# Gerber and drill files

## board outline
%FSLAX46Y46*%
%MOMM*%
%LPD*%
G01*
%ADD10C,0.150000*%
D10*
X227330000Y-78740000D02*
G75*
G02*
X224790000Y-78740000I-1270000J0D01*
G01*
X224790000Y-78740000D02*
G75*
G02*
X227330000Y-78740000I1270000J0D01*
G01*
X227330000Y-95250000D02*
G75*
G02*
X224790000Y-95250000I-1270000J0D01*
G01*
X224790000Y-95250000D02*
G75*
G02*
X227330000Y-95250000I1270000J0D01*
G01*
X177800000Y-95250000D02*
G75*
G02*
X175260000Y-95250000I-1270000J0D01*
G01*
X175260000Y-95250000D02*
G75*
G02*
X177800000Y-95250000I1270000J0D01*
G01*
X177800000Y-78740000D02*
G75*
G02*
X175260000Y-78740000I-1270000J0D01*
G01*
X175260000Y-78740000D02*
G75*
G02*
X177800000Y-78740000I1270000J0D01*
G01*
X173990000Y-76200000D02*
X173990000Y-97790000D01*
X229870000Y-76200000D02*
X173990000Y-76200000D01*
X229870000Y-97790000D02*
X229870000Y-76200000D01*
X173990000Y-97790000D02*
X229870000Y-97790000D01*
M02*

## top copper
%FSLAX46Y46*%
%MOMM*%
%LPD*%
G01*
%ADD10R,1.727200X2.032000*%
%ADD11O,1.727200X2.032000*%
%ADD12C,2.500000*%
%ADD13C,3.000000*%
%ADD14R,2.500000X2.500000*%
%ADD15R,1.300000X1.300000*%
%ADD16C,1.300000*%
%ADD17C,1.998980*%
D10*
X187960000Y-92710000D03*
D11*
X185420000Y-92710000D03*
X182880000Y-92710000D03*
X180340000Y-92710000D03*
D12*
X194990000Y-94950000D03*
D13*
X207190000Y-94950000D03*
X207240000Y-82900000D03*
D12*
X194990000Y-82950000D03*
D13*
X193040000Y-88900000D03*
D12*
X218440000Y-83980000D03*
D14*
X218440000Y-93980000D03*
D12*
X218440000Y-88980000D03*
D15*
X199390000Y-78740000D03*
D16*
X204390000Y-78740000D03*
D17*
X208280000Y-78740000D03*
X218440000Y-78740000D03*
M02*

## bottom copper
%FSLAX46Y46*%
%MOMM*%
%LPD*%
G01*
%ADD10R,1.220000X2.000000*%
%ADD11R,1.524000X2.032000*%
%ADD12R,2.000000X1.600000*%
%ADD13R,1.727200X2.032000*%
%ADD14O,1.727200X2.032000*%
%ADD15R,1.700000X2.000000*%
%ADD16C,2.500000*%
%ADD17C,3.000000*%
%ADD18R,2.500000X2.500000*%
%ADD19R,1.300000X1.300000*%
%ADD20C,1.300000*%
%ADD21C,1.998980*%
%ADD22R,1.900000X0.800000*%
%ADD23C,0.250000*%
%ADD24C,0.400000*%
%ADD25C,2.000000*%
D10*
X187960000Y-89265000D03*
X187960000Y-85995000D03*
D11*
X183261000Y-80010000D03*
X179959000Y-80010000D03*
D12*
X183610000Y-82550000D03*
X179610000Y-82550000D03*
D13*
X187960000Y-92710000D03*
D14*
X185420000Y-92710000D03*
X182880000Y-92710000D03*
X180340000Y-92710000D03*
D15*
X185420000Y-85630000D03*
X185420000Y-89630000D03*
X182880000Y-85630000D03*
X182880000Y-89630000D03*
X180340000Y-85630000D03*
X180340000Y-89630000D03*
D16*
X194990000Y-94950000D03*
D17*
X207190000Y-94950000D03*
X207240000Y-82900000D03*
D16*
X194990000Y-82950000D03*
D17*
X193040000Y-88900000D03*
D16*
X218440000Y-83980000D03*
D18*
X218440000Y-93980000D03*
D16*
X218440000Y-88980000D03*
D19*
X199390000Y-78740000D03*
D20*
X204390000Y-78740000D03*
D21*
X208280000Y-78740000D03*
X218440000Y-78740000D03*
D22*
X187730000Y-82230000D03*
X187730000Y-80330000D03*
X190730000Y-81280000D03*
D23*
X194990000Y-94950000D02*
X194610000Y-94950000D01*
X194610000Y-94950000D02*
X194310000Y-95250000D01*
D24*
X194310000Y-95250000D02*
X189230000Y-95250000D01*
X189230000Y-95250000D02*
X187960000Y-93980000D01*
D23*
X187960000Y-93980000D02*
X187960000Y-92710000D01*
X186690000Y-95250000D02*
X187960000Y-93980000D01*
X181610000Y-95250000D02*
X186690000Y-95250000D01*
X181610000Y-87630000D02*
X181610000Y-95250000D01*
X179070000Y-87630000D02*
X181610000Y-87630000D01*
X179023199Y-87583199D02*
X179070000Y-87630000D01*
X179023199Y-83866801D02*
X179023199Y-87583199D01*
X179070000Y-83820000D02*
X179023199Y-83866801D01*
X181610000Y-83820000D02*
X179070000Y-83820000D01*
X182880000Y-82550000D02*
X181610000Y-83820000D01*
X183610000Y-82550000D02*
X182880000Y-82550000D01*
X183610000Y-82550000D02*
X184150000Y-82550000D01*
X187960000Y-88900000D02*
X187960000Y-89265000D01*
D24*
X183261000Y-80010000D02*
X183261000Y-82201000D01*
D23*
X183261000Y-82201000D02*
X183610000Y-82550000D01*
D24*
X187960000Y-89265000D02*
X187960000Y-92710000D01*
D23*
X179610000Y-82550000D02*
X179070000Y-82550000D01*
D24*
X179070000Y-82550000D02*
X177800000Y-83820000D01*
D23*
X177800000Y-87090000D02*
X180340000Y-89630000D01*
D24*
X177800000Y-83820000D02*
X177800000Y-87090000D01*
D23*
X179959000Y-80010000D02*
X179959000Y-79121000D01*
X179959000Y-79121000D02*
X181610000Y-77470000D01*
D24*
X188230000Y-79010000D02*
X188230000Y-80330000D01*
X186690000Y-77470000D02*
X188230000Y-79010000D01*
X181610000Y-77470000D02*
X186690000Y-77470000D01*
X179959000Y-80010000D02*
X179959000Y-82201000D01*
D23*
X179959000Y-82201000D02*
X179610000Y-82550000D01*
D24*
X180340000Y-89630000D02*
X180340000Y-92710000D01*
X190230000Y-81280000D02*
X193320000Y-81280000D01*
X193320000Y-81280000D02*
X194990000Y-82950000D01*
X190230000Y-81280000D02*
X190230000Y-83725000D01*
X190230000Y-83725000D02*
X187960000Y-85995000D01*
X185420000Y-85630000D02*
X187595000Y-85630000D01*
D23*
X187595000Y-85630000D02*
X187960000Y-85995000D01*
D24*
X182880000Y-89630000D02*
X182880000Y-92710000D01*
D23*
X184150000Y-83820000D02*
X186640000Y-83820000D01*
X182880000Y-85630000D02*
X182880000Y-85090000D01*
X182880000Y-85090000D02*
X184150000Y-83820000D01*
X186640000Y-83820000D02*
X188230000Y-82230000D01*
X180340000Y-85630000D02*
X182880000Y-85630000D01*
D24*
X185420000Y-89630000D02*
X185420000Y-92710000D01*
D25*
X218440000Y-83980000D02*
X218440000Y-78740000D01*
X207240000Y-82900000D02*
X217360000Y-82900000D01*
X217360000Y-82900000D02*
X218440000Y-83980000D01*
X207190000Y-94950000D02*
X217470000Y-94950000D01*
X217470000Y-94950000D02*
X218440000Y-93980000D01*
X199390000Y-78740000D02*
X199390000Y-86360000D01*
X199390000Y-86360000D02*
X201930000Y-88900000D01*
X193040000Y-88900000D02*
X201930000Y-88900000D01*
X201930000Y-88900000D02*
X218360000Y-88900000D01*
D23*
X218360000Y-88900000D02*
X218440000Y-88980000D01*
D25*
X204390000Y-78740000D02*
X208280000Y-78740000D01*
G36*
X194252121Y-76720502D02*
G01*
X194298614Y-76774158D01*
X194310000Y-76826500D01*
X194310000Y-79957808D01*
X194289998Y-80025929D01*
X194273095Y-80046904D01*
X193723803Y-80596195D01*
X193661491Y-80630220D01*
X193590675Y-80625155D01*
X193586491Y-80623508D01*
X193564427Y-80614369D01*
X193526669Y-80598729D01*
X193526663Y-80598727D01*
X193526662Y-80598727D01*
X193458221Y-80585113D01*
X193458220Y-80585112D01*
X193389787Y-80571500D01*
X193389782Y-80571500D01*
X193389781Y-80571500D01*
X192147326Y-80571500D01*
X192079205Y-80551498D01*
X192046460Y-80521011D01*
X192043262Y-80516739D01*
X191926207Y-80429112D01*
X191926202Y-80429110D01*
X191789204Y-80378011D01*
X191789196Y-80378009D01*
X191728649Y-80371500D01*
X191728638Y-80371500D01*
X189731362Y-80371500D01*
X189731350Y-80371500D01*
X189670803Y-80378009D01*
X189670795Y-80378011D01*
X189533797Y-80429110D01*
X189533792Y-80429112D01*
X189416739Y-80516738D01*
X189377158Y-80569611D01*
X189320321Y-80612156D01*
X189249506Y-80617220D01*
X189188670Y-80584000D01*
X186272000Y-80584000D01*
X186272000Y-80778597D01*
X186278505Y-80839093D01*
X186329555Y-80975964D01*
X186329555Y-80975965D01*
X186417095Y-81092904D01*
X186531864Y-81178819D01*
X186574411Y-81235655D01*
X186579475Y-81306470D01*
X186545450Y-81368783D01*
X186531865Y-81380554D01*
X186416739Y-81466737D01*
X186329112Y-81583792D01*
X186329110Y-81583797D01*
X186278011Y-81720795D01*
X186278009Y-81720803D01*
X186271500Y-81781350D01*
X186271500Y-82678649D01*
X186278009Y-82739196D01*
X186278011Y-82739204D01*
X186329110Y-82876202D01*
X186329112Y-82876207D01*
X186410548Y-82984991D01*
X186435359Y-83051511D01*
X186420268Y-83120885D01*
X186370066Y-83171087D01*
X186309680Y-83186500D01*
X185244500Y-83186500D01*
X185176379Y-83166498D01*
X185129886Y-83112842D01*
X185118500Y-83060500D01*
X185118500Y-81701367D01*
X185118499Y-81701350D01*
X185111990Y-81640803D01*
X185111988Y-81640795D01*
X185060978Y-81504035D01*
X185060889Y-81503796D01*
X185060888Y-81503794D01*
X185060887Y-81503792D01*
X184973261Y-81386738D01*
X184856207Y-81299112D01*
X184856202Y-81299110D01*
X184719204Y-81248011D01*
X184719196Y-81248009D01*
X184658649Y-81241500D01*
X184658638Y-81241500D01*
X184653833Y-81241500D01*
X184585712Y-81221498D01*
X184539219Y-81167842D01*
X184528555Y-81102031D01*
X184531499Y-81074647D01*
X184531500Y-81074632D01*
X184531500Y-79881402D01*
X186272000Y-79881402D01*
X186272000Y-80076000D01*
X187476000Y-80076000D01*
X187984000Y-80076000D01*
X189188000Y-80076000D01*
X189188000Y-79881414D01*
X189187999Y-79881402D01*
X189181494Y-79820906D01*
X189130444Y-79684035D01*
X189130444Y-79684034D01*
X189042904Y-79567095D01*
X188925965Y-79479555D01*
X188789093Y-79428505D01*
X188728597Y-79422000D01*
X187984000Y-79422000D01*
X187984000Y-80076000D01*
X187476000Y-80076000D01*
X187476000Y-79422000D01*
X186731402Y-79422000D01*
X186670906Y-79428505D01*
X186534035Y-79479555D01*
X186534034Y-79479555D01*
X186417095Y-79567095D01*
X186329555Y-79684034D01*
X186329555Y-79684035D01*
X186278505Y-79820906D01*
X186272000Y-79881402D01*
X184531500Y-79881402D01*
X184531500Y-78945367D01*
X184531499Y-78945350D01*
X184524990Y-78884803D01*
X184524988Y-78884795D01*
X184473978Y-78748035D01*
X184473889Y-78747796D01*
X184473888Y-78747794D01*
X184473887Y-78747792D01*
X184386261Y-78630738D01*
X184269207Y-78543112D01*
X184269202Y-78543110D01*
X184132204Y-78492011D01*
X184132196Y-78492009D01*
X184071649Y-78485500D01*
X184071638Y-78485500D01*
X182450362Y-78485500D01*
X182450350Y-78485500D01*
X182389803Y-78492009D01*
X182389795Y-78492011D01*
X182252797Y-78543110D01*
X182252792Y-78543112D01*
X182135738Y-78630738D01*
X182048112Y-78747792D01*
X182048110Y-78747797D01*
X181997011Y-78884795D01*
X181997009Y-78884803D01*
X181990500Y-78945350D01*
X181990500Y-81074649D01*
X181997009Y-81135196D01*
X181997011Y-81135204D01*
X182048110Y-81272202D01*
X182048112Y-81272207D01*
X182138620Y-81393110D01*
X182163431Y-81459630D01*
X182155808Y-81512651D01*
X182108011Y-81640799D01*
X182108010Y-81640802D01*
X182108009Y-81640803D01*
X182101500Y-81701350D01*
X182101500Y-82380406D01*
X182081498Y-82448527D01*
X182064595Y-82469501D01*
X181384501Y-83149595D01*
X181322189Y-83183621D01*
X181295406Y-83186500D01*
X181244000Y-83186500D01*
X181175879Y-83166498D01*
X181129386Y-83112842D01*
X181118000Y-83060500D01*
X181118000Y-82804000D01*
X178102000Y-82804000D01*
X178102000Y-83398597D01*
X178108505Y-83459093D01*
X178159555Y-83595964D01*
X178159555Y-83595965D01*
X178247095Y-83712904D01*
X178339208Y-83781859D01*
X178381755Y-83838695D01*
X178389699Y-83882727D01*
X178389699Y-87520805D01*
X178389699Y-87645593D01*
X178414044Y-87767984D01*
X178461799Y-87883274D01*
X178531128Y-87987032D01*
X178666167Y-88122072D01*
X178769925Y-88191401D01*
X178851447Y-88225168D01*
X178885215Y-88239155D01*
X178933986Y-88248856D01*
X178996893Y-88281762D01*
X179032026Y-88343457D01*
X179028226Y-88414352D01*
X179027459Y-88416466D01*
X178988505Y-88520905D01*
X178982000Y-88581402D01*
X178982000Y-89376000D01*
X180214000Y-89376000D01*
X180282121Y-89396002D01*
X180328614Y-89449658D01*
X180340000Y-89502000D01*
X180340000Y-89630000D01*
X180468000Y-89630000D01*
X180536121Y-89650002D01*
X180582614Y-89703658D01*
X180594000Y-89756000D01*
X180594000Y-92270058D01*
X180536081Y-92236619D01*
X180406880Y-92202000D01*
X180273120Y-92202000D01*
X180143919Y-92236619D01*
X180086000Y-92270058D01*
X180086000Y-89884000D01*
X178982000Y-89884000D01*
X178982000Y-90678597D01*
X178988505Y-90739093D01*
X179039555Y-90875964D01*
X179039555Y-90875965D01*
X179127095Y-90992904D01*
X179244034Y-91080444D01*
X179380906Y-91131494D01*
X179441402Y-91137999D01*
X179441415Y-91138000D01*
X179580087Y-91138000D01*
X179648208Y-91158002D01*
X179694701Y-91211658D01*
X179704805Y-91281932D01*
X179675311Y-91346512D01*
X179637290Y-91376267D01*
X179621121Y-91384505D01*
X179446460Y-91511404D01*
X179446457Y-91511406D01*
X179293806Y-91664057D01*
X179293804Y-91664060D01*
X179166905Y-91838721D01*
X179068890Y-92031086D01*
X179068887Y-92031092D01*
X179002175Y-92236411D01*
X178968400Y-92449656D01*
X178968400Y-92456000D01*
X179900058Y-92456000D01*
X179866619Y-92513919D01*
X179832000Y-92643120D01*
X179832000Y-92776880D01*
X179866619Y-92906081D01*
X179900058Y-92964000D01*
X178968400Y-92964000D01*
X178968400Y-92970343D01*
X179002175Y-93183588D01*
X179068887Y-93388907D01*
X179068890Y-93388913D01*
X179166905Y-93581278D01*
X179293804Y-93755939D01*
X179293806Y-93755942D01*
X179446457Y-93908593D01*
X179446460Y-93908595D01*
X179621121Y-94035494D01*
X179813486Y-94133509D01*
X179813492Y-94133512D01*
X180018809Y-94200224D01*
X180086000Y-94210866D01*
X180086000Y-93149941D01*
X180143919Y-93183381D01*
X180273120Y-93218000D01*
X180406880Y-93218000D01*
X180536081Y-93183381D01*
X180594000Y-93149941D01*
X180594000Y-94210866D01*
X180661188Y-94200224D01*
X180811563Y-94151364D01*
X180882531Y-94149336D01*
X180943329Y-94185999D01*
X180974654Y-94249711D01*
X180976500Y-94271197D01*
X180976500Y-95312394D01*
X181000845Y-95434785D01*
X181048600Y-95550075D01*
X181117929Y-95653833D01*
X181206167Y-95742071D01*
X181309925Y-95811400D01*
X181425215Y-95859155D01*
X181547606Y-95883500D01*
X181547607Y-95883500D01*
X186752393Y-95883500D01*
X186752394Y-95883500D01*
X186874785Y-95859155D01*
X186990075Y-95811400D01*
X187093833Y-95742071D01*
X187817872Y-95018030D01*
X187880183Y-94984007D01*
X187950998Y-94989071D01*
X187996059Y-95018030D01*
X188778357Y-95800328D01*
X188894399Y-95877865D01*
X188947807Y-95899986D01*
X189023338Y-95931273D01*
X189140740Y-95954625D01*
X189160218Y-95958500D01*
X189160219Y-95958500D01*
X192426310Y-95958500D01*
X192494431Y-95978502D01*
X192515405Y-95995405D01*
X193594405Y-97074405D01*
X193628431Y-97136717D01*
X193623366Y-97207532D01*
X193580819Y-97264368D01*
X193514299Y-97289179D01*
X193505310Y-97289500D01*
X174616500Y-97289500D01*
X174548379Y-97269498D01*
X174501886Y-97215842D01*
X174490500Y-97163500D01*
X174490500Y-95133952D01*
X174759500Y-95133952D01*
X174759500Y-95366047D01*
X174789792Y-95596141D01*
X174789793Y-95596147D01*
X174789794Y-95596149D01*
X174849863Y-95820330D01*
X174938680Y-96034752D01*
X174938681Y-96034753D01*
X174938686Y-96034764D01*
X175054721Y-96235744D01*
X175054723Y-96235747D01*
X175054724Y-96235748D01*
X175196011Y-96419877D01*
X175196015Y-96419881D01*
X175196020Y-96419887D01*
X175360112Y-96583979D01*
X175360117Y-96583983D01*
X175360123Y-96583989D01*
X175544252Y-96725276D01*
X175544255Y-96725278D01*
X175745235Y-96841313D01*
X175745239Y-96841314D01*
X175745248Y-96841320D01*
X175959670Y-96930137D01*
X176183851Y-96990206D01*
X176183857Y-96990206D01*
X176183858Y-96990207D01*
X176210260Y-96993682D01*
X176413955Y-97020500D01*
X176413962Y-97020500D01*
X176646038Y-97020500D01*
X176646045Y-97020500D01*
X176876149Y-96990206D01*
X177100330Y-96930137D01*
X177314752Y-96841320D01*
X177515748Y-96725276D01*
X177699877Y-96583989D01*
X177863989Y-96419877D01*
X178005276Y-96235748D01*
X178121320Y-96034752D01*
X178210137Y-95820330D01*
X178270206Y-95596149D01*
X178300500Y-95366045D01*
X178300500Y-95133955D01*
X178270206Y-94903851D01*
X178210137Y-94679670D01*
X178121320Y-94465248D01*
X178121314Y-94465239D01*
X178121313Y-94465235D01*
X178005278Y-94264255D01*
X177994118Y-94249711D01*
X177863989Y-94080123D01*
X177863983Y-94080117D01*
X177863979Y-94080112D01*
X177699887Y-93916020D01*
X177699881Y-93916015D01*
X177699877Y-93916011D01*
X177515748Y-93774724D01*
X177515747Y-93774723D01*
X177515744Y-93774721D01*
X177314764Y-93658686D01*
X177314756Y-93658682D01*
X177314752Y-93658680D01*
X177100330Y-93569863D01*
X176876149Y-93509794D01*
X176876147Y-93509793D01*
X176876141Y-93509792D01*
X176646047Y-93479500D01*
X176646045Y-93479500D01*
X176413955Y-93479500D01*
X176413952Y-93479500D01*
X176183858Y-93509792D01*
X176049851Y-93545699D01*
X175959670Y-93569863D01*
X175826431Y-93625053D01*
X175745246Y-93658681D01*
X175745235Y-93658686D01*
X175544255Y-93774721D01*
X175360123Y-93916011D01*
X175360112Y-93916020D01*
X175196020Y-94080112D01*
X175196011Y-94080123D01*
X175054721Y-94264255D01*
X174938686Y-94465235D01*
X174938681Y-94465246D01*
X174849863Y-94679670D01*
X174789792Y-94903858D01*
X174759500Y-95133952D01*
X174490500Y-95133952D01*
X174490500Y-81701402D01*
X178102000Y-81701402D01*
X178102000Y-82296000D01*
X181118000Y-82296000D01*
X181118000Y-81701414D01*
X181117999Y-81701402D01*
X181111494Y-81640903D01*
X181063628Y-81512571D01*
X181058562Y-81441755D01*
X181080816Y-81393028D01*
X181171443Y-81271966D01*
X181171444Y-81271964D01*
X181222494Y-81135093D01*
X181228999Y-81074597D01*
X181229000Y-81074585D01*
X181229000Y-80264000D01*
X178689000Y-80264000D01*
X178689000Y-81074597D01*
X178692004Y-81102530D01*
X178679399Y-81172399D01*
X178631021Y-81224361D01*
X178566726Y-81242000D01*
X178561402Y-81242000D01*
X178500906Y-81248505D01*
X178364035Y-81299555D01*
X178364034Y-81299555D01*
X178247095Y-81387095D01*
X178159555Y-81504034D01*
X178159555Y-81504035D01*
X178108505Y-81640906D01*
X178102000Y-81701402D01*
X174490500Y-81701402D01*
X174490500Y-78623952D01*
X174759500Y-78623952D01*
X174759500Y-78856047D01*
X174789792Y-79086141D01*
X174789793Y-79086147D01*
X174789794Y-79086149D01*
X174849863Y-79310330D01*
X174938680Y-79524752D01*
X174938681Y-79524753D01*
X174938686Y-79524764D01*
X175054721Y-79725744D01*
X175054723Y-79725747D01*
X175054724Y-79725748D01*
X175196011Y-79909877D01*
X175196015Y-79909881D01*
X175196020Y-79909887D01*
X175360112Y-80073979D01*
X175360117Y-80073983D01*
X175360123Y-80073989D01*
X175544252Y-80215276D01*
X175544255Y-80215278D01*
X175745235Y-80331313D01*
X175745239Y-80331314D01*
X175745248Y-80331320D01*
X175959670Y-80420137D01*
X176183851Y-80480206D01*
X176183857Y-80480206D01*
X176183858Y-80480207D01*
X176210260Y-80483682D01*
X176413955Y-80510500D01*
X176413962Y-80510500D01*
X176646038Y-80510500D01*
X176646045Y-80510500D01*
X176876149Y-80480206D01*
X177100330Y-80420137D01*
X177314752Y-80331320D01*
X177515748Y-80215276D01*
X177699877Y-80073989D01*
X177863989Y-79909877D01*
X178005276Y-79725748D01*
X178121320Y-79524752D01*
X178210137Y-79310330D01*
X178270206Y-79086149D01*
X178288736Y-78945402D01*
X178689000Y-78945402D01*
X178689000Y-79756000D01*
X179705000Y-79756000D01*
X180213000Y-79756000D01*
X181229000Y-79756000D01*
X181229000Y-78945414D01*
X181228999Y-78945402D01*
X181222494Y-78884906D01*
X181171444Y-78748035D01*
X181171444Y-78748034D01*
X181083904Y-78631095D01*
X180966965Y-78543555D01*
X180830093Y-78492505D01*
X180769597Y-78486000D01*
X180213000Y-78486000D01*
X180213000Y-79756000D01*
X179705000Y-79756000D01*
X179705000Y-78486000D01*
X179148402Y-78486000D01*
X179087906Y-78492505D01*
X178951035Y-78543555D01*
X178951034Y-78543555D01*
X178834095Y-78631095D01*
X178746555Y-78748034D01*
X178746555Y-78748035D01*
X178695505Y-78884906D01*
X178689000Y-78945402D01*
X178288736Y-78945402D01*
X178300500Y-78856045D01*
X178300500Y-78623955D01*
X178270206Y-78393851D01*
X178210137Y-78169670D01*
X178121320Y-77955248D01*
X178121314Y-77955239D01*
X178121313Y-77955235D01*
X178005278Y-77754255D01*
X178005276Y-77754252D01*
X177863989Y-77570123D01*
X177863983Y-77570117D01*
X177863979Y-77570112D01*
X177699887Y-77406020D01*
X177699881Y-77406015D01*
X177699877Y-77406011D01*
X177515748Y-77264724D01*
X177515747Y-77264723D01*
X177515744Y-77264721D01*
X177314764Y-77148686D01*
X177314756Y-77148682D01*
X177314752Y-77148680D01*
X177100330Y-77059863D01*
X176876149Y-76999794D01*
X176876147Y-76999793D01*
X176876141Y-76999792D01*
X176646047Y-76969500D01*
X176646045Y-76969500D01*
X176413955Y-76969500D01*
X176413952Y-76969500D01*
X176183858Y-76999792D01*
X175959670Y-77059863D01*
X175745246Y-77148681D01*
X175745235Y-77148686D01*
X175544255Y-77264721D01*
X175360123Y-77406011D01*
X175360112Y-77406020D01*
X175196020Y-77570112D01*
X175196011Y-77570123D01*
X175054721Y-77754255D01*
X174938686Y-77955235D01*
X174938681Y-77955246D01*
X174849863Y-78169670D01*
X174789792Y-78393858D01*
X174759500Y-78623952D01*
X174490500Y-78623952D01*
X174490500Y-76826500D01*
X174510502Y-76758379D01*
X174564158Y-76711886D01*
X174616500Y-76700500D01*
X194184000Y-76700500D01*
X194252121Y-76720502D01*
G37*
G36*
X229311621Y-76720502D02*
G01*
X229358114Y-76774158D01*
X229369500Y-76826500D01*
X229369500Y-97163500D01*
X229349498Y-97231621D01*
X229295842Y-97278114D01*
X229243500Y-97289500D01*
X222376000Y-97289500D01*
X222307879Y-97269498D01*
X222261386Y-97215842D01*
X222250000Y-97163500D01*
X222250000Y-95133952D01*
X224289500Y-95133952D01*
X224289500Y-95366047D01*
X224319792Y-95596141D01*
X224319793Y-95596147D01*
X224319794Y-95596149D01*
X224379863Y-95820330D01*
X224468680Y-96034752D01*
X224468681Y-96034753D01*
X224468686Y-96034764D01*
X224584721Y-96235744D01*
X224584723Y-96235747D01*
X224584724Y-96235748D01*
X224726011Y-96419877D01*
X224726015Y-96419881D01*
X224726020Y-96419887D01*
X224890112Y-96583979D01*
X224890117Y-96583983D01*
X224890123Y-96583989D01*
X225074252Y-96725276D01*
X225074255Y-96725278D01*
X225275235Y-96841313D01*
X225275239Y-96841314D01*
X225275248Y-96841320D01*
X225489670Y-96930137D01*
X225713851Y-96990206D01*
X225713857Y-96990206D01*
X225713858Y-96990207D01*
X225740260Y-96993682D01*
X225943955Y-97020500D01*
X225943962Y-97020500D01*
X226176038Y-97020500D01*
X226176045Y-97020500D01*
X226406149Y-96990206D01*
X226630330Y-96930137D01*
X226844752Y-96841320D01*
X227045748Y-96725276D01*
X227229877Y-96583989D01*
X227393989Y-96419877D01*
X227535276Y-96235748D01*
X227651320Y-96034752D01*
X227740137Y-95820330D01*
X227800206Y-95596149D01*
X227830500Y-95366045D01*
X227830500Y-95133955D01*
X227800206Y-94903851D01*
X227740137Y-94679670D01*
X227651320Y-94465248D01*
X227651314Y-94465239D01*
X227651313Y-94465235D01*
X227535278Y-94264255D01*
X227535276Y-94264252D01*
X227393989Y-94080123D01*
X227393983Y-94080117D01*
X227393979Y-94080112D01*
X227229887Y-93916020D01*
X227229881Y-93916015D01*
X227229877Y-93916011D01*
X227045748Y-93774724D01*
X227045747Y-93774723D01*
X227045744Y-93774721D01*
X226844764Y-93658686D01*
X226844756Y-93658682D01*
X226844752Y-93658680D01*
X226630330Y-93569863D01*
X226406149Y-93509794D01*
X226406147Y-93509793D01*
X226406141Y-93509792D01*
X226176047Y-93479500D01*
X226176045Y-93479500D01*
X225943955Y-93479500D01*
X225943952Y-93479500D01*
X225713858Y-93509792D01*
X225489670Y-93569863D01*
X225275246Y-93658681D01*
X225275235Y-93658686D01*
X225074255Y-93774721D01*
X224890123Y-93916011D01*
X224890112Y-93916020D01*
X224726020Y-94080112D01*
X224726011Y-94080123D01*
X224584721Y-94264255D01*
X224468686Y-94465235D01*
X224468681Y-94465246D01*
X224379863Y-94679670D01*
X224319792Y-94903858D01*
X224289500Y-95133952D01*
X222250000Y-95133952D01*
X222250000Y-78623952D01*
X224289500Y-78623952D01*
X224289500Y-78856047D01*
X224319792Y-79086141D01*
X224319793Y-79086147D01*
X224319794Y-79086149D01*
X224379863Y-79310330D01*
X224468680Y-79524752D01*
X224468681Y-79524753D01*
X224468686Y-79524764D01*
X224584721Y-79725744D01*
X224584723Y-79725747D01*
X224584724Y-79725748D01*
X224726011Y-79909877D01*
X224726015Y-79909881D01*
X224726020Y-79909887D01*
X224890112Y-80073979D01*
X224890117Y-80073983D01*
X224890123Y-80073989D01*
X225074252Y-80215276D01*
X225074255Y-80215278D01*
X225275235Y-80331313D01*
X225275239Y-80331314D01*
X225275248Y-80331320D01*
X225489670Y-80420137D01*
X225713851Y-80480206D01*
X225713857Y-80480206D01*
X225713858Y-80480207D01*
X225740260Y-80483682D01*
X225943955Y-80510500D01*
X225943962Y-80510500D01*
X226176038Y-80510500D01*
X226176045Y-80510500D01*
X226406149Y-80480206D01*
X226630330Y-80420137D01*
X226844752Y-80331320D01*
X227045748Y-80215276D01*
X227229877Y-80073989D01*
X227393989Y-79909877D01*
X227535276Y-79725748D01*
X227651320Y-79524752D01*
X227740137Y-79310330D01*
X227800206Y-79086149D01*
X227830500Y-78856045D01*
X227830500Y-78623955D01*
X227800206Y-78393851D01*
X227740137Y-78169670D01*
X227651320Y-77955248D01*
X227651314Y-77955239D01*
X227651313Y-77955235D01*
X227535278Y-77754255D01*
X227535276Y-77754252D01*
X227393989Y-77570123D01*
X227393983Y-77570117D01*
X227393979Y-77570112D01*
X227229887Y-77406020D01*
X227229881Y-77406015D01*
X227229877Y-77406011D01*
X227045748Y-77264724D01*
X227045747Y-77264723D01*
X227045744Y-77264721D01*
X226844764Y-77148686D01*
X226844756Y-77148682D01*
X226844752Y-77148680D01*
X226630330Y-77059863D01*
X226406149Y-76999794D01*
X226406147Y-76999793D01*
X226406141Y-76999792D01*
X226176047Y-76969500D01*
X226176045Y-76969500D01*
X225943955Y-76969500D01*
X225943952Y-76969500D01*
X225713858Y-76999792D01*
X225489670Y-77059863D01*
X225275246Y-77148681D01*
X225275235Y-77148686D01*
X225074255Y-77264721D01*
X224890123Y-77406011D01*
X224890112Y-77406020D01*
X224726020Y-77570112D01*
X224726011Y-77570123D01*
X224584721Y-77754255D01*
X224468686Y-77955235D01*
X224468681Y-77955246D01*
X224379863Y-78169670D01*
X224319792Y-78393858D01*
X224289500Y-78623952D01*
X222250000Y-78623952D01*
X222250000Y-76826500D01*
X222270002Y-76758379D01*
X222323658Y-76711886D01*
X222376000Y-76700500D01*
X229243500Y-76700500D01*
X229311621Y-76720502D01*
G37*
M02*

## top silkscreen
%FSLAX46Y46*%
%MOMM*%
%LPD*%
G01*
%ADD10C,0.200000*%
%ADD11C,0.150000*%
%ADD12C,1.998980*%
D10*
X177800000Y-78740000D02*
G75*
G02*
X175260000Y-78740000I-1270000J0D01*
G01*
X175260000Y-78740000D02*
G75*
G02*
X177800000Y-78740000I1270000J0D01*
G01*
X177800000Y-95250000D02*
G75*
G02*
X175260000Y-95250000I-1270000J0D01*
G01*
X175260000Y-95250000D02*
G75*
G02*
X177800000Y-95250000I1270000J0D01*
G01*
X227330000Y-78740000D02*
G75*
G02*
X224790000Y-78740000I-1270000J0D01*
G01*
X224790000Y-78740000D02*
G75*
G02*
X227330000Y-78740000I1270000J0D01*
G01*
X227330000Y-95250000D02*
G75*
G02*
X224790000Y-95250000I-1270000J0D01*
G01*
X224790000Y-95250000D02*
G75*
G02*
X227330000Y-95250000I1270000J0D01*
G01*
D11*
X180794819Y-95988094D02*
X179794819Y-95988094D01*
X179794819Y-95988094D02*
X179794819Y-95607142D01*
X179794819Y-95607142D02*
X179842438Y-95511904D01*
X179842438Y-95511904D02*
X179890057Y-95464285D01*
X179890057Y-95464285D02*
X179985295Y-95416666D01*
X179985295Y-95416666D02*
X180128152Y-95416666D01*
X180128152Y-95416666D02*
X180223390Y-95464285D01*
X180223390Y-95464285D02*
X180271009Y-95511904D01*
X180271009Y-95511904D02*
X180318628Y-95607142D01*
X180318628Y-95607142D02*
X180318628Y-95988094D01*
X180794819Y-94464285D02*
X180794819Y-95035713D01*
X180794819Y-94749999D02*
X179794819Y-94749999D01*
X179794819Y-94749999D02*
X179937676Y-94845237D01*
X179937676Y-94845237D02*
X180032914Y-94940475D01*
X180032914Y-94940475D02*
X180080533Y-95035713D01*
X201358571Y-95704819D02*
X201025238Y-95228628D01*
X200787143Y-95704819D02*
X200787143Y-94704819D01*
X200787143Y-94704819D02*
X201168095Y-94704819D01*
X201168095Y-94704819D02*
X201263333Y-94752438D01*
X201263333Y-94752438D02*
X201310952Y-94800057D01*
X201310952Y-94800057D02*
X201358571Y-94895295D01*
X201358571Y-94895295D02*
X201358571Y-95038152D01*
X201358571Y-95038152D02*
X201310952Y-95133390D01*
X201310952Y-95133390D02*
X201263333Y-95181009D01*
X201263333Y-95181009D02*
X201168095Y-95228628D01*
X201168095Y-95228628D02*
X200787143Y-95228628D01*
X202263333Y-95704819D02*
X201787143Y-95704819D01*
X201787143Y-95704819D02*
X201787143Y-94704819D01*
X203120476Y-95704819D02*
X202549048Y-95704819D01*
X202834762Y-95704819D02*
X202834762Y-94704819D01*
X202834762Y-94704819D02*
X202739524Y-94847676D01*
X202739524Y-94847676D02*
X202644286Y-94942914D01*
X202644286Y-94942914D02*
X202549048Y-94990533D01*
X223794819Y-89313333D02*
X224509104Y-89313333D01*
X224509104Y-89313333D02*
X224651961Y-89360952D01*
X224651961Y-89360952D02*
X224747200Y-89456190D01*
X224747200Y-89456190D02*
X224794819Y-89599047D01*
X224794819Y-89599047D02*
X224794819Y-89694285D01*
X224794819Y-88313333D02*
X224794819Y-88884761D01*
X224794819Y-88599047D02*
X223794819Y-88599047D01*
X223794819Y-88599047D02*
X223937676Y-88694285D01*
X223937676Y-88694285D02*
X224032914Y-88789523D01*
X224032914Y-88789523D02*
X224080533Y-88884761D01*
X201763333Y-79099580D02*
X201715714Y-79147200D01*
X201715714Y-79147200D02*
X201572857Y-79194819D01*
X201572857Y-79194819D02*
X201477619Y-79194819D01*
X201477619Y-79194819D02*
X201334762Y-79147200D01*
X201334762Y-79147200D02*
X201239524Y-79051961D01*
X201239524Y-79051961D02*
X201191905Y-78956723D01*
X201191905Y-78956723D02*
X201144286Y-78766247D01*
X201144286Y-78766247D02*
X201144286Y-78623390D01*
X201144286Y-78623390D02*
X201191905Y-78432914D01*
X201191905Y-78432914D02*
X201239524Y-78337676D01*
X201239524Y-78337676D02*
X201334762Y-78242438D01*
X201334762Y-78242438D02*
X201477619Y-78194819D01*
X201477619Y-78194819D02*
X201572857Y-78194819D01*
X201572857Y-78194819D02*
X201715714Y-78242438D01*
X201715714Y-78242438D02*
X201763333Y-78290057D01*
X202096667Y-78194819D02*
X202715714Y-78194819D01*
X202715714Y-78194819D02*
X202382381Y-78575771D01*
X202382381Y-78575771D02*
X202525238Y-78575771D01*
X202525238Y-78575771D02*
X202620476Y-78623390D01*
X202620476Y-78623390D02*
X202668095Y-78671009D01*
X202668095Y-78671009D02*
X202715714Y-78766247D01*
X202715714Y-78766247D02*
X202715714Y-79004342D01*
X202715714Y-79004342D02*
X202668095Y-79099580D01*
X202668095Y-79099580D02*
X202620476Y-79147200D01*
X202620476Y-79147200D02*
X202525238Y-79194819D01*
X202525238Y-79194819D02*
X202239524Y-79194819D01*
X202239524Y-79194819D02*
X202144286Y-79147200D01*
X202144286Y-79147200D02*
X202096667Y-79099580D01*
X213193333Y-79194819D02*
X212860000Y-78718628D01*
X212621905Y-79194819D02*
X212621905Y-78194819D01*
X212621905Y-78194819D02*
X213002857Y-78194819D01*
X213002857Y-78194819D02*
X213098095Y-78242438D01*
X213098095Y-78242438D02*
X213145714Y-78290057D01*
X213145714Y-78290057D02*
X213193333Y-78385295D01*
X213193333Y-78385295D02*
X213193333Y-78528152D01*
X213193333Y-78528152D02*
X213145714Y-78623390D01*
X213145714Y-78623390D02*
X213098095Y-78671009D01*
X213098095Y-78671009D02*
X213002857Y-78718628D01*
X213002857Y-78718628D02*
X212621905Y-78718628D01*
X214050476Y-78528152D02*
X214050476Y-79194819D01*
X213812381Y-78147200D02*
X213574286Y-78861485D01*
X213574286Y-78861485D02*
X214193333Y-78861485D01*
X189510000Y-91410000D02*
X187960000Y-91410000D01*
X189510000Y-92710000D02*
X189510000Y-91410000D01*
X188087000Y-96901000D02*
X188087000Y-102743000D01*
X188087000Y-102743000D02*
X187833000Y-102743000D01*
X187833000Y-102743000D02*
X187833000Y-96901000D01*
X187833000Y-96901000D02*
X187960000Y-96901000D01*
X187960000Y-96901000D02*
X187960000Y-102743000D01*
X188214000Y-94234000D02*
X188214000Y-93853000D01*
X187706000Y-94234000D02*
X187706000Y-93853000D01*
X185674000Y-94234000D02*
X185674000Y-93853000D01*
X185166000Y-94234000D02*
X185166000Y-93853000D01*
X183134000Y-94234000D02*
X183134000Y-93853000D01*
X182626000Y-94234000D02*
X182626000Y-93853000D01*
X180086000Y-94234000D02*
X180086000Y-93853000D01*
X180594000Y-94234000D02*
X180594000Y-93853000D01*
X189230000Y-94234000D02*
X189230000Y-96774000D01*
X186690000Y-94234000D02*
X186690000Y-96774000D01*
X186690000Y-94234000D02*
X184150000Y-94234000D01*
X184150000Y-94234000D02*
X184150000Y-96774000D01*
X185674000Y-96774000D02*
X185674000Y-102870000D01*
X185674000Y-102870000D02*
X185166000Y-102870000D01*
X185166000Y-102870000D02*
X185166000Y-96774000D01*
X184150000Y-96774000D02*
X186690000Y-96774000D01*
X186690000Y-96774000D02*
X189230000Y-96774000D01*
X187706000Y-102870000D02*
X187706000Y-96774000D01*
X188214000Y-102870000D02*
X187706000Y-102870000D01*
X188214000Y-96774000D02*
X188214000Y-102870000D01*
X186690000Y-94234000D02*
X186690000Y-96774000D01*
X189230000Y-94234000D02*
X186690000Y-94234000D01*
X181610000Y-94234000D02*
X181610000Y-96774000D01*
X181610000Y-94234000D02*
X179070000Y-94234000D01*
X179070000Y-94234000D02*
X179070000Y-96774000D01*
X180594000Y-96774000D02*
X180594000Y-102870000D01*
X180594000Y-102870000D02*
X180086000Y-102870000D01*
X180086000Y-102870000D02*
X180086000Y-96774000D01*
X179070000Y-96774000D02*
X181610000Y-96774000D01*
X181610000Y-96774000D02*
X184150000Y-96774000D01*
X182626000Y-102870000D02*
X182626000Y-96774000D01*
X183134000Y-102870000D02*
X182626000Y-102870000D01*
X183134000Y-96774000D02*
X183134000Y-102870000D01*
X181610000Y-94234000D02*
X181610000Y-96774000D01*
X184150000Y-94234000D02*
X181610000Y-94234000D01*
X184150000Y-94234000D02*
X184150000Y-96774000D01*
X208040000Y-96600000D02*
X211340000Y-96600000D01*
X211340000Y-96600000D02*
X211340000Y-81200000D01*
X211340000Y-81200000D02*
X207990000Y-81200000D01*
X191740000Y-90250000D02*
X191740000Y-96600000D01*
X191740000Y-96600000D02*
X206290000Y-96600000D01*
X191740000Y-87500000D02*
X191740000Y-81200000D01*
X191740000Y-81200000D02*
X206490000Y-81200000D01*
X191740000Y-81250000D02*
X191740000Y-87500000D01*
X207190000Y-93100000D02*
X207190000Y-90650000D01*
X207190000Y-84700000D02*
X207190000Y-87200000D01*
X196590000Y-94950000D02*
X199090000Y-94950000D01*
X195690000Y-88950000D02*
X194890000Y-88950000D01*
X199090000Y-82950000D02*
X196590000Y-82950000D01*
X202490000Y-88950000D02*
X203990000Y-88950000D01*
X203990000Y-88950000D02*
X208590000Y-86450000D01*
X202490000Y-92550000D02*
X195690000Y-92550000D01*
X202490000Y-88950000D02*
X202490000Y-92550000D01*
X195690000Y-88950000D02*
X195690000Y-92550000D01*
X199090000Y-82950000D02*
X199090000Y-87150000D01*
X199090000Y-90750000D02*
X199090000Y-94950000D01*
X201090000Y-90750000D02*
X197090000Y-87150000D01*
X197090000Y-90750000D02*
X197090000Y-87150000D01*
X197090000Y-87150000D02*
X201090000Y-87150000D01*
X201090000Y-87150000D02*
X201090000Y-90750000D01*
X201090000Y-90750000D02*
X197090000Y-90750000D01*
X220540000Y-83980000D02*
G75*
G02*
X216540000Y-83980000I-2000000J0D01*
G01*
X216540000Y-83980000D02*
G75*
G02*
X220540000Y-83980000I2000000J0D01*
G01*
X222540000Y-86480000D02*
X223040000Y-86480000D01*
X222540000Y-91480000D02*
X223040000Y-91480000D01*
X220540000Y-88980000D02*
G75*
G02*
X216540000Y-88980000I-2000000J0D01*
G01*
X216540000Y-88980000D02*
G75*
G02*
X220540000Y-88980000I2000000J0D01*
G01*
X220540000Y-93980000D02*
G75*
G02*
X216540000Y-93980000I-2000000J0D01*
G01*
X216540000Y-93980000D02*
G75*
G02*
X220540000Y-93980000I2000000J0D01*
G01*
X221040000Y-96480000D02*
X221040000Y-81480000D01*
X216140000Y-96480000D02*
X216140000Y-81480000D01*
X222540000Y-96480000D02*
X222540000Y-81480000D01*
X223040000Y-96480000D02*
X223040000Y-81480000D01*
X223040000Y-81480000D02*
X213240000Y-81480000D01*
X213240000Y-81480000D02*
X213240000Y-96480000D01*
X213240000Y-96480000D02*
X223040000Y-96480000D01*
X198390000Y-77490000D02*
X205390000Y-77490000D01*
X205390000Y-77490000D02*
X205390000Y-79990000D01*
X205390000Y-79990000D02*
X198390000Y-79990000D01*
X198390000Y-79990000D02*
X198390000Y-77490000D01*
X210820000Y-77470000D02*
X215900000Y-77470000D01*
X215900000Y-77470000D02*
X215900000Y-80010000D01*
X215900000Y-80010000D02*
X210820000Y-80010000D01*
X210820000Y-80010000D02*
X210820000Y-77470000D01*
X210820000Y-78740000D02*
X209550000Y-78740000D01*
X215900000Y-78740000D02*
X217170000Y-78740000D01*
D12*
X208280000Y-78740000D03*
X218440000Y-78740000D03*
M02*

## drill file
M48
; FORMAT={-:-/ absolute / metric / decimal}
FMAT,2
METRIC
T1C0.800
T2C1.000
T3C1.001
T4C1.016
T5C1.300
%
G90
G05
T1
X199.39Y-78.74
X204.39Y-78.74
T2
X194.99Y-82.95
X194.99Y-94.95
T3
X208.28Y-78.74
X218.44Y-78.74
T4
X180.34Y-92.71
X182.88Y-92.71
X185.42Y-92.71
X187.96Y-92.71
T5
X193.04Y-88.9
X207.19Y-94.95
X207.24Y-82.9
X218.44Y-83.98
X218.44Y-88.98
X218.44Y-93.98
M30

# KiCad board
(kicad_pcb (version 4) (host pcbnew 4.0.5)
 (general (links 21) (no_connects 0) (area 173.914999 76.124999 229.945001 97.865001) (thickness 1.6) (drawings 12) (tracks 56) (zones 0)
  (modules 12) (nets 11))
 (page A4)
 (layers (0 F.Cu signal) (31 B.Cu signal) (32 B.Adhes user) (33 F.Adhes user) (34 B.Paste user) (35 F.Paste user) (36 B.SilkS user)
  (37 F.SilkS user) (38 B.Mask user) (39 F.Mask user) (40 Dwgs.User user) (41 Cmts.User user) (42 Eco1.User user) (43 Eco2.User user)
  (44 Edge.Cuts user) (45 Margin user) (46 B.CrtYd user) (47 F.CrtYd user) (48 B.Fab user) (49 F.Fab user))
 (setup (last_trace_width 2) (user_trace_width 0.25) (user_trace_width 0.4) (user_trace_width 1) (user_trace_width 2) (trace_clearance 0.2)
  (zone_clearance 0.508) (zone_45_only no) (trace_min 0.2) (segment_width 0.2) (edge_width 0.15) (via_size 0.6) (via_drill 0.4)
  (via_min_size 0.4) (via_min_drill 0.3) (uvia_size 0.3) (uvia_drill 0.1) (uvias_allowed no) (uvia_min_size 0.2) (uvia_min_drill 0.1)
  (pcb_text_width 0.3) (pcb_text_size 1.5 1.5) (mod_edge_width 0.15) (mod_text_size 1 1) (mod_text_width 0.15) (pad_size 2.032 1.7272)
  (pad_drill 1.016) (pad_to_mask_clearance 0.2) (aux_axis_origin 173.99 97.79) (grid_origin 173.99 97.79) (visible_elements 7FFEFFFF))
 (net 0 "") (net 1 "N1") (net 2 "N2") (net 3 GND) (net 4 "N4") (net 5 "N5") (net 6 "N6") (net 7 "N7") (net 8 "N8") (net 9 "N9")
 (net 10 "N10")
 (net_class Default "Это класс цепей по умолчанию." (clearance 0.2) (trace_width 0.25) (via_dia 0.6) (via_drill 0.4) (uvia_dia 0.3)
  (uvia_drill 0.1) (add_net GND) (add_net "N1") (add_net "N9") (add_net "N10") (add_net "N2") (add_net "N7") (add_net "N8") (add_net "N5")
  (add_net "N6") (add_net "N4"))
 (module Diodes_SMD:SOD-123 (layer B.Cu) (at 187.96 87.63 90)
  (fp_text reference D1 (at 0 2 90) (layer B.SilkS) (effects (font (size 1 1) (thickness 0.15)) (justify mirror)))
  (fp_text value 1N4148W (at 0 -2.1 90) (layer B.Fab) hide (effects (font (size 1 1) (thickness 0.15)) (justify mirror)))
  (pad 1 smd rect (at -1.635 0 90) (size 2 1.22) (layers B.Cu B.Paste B.Mask) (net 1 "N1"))
  (pad 2 smd rect (at 1.635 0 90) (size 2 1.22) (layers B.Cu B.Paste B.Mask) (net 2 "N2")))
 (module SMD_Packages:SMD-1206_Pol (layer B.Cu) (at 181.61 80.01 180)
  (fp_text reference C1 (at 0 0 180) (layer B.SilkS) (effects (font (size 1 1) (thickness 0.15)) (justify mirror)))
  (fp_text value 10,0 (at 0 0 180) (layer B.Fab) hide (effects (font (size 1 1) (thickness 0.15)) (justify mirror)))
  (pad 1 smd rect (at -1.651 0 180) (size 1.524 2.032) (layers B.Cu B.Paste B.Mask) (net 1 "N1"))
  (pad 2 smd rect (at 1.651 0 180) (size 1.524 2.032) (layers B.Cu B.Paste B.Mask) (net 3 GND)))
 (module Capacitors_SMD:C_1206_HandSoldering (layer B.Cu) (at 181.61 82.55 180)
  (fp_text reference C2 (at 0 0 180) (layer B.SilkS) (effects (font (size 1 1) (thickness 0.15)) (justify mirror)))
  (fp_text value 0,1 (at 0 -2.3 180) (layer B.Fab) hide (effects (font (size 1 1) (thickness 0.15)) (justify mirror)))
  (pad 1 smd rect (at -2 0 180) (size 2 1.6) (layers B.Cu B.Paste B.Mask) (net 1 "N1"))
  (pad 2 smd rect (at 2 0 180) (size 2 1.6) (layers B.Cu B.Paste B.Mask) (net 3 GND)))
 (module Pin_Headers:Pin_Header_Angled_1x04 (layer F.Cu) (at 187.96 92.71 270)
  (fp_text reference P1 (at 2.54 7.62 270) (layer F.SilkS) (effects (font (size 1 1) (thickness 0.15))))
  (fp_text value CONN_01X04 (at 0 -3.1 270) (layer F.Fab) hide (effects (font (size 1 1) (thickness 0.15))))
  (fp_line (start -1.3 -1.55) (end -1.3 0) (layer F.SilkS) (width 0.15))
  (fp_line (start 0 -1.55) (end -1.3 -1.55) (layer F.SilkS) (width 0.15))
  (fp_line (start 4.191 -0.127) (end 10.033 -0.127) (layer F.SilkS) (width 0.15))
  (fp_line (start 10.033 -0.127) (end 10.033 0.127) (layer F.SilkS) (width 0.15))
  (fp_line (start 10.033 0.127) (end 4.191 0.127) (layer F.SilkS) (width 0.15))
  (fp_line (start 4.191 0.127) (end 4.191 0) (layer F.SilkS) (width 0.15))
  (fp_line (start 4.191 0) (end 10.033 0) (layer F.SilkS) (width 0.15))
  (fp_line (start 1.524 -0.254) (end 1.143 -0.254) (layer F.SilkS) (width 0.15))
  (fp_line (start 1.524 0.254) (end 1.143 0.254) (layer F.SilkS) (width 0.15))
  (fp_line (start 1.524 2.286) (end 1.143 2.286) (layer F.SilkS) (width 0.15))
  (fp_line (start 1.524 2.794) (end 1.143 2.794) (layer F.SilkS) (width 0.15))
  (fp_line (start 1.524 4.826) (end 1.143 4.826) (layer F.SilkS) (width 0.15))
  (fp_line (start 1.524 5.334) (end 1.143 5.334) (layer F.SilkS) (width 0.15))
  (fp_line (start 1.524 7.874) (end 1.143 7.874) (layer F.SilkS) (width 0.15))
  (fp_line (start 1.524 7.366) (end 1.143 7.366) (layer F.SilkS) (width 0.15))
  (fp_line (start 1.524 -1.27) (end 4.064 -1.27) (layer F.SilkS) (width 0.15))
  (fp_line (start 1.524 1.27) (end 4.064 1.27) (layer F.SilkS) (width 0.15))
  (fp_line (start 1.524 1.27) (end 1.524 3.81) (layer F.SilkS) (width 0.15))
  (fp_line (start 1.524 3.81) (end 4.064 3.81) (layer F.SilkS) (width 0.15))
  (fp_line (start 4.064 2.286) (end 10.16 2.286) (layer F.SilkS) (width 0.15))
  (fp_line (start 10.16 2.286) (end 10.16 2.794) (layer F.SilkS) (width 0.15))
  (fp_line (start 10.16 2.794) (end 4.064 2.794) (layer F.SilkS) (width 0.15))
  (fp_line (start 4.064 3.81) (end 4.064 1.27) (layer F.SilkS) (width 0.15))
  (fp_line (start 4.064 1.27) (end 4.064 -1.27) (layer F.SilkS) (width 0.15))
  (fp_line (start 10.16 0.254) (end 4.064 0.254) (layer F.SilkS) (width 0.15))
  (fp_line (start 10.16 -0.254) (end 10.16 0.254) (layer F.SilkS) (width 0.15))
  (fp_line (start 4.064 -0.254) (end 10.16 -0.254) (layer F.SilkS) (width 0.15))
  (fp_line (start 1.524 1.27) (end 4.064 1.27) (layer F.SilkS) (width 0.15))
  (fp_line (start 1.524 -1.27) (end 1.524 1.27) (layer F.SilkS) (width 0.15))
  (fp_line (start 1.524 6.35) (end 4.064 6.35) (layer F.SilkS) (width 0.15))
  (fp_line (start 1.524 6.35) (end 1.524 8.89) (layer F.SilkS) (width 0.15))
  (fp_line (start 1.524 8.89) (end 4.064 8.89) (layer F.SilkS) (width 0.15))
  (fp_line (start 4.064 7.366) (end 10.16 7.366) (layer F.SilkS) (width 0.15))
  (fp_line (start 10.16 7.366) (end 10.16 7.874) (layer F.SilkS) (width 0.15))
  (fp_line (start 10.16 7.874) (end 4.064 7.874) (layer F.SilkS) (width 0.15))
  (fp_line (start 4.064 8.89) (end 4.064 6.35) (layer F.SilkS) (width 0.15))
  (fp_line (start 4.064 6.35) (end 4.064 3.81) (layer F.SilkS) (width 0.15))
  (fp_line (start 10.16 5.334) (end 4.064 5.334) (layer F.SilkS) (width 0.15))
  (fp_line (start 10.16 4.826) (end 10.16 5.334) (layer F.SilkS) (width 0.15))
  (fp_line (start 4.064 4.826) (end 10.16 4.826) (layer F.SilkS) (width 0.15))
  (fp_line (start 1.524 6.35) (end 4.064 6.35) (layer F.SilkS) (width 0.15))
  (fp_line (start 1.524 3.81) (end 1.524 6.35) (layer F.SilkS) (width 0.15))
  (fp_line (start 1.524 3.81) (end 4.064 3.81) (layer F.SilkS) (width 0.15))
  (pad 1 thru_hole rect (at 0 0 270) (size 2.032 1.7272) (drill 1.016) (layers *.Cu *.Mask) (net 1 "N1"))
  (pad 2 thru_hole oval (at 0 2.54 270) (size 2.032 1.7272) (drill 1.016) (layers *.Cu *.Mask) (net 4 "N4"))
  (pad 3 thru_hole oval (at 0 5.08 270) (size 2.032 1.7272) (drill 1.016) (layers *.Cu *.Mask) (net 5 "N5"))
  (pad 4 thru_hole oval (at 0 7.62 270) (size 2.032 1.7272) (drill 1.016) (layers *.Cu *.Mask) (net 3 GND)))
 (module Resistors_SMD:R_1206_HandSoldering (layer B.Cu) (at 185.42 87.63 270)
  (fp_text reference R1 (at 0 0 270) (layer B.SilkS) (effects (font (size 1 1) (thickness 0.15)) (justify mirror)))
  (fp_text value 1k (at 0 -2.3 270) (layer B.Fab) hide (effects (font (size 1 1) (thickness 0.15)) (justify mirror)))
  (pad 1 smd rect (at -2 0 270) (size 2 1.7) (layers B.Cu B.Paste B.Mask) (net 2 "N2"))
  (pad 2 smd rect (at 2 0 270) (size 2 1.7) (layers B.Cu B.Paste B.Mask) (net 4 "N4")))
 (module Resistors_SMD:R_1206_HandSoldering (layer B.Cu) (at 182.88 87.63 270)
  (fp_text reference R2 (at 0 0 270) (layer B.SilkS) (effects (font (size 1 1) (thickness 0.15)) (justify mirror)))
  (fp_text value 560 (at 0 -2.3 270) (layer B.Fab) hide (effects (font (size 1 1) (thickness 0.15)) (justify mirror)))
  (pad 1 smd rect (at -2 0 270) (size 2 1.7) (layers B.Cu B.Paste B.Mask) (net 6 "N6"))
  (pad 2 smd rect (at 2 0 270) (size 2 1.7) (layers B.Cu B.Paste B.Mask) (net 5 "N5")))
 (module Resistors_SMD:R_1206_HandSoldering (layer B.Cu) (at 180.34 87.63 270)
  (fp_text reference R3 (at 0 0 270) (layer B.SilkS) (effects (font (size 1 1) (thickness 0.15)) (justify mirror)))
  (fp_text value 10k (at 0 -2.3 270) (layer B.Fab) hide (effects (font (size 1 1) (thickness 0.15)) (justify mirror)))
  (pad 1 smd rect (at -2 0 270) (size 2 1.7) (layers B.Cu B.Paste B.Mask) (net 6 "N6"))
  (pad 2 smd rect (at 2 0 270) (size 2 1.7) (layers B.Cu B.Paste B.Mask) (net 3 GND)))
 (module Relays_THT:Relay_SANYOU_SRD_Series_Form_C (layer F.Cu) (at 193.04 88.9)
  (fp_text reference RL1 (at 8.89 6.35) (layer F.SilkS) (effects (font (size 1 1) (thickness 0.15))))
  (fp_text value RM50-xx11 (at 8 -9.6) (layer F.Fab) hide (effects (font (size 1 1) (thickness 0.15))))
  (fp_line (start 15 7.7) (end 18.3 7.7) (layer F.SilkS) (width 0.15))
  (fp_line (start 18.3 7.7) (end 18.3 -7.7) (layer F.SilkS) (width 0.15))
  (fp_line (start 18.3 -7.7) (end 14.95 -7.7) (layer F.SilkS) (width 0.15))
  (fp_line (start -1.3 1.35) (end -1.3 7.7) (layer F.SilkS) (width 0.15))
  (fp_line (start -1.3 7.7) (end 13.25 7.7) (layer F.SilkS) (width 0.15))
  (fp_line (start -1.3 -1.4) (end -1.3 -7.7) (layer F.SilkS) (width 0.15))
  (fp_line (start -1.3 -7.7) (end 13.45 -7.7) (layer F.SilkS) (width 0.15))
  (fp_line (start -1.3 -7.65) (end -1.3 -1.4) (layer F.SilkS) (width 0.15))
  (fp_line (start 14.15 4.2) (end 14.15 1.75) (layer F.SilkS) (width 0.15))
  (fp_line (start 14.15 -4.2) (end 14.15 -1.7) (layer F.SilkS) (width 0.15))
  (fp_line (start 3.55 6.05) (end 6.05 6.05) (layer F.SilkS) (width 0.15))
  (fp_line (start 2.65 0.05) (end 1.85 0.05) (layer F.SilkS) (width 0.15))
  (fp_line (start 6.05 -5.95) (end 3.55 -5.95) (layer F.SilkS) (width 0.15))
  (fp_line (start 9.45 0.05) (end 10.95 0.05) (layer F.SilkS) (width 0.15))
  (fp_line (start 10.95 0.05) (end 15.55 -2.45) (layer F.SilkS) (width 0.15))
  (fp_line (start 9.45 3.65) (end 2.65 3.65) (layer F.SilkS) (width 0.15))
  (fp_line (start 9.45 0.05) (end 9.45 3.65) (layer F.SilkS) (width 0.15))
  (fp_line (start 2.65 0.05) (end 2.65 3.65) (layer F.SilkS) (width 0.15))
  (fp_line (start 6.05 -5.95) (end 6.05 -1.75) (layer F.SilkS) (width 0.15))
  (fp_line (start 6.05 1.85) (end 6.05 6.05) (layer F.SilkS) (width 0.15))
  (fp_line (start 8.05 1.85) (end 4.05 -1.75) (layer F.SilkS) (width 0.15))
  (fp_line (start 4.05 1.85) (end 4.05 -1.75) (layer F.SilkS) (width 0.15))
  (fp_line (start 4.05 -1.75) (end 8.05 -1.75) (layer F.SilkS) (width 0.15))
  (fp_line (start 8.05 -1.75) (end 8.05 1.85) (layer F.SilkS) (width 0.15))
  (fp_line (start 8.05 1.85) (end 4.05 1.85) (layer F.SilkS) (width 0.15))
  (pad 2 thru_hole circle (at 1.95 6.05 90) (size 2.5 2.5) (drill 1) (layers *.Cu *.Mask) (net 1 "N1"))
  (pad 3 thru_hole circle (at 14.15 6.05 90) (size 3 3) (drill 1.3) (layers *.Cu *.Mask) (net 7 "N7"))
  (pad 4 thru_hole circle (at 14.2 -6 90) (size 3 3) (drill 1.3) (layers *.Cu *.Mask) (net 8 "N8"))
  (pad 5 thru_hole circle (at 1.95 -5.95 90) (size 2.5 2.5) (drill 1) (layers *.Cu *.Mask) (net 2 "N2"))
  (pad 1 thru_hole circle (at 0 0 90) (size 3 3) (drill 1.3) (layers *.Cu *.Mask) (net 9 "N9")))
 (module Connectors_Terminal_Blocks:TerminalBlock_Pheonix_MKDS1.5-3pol (layer F.Cu) (at 218.44 93.98 90)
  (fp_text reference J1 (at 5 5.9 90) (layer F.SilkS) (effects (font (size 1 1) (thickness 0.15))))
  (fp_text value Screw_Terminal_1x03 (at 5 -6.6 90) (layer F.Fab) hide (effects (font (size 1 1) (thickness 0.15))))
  (fp_circle (center 10 0.1) (end 8 0.1) (layer F.SilkS) (width 0.15))
  (fp_line (start 7.5 4.1) (end 7.5 4.6) (layer F.SilkS) (width 0.15))
  (fp_line (start 2.5 4.1) (end 2.5 4.6) (layer F.SilkS) (width 0.15))
  (fp_circle (center 5 0.1) (end 3 0.1) (layer F.SilkS) (width 0.15))
  (fp_circle (center 0 0.1) (end 2 0.1) (layer F.SilkS) (width 0.15))
  (fp_line (start -2.5 2.6) (end 12.5 2.6) (layer F.SilkS) (width 0.15))
  (fp_line (start -2.5 -2.3) (end 12.5 -2.3) (layer F.SilkS) (width 0.15))
  (fp_line (start -2.5 4.1) (end 12.5 4.1) (layer F.SilkS) (width 0.15))
  (fp_line (start -2.5 4.6) (end 12.5 4.6) (layer F.SilkS) (width 0.15))
  (fp_line (start 12.5 4.6) (end 12.5 -5.2) (layer F.SilkS) (width 0.15))
  (fp_line (start 12.5 -5.2) (end -2.5 -5.2) (layer F.SilkS) (width 0.15))
  (fp_line (start -2.5 -5.2) (end -2.5 4.6) (layer F.SilkS) (width 0.15))
  (pad 3 thru_hole circle (at 10 0 90) (size 2.5 2.5) (drill 1.3) (layers *.Cu *.Mask) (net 8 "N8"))
  (pad 1 thru_hole rect (at 0 0 90) (size 2.5 2.5) (drill 1.3) (layers *.Cu *.Mask) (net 7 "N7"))
  (pad 2 thru_hole circle (at 5 0 90) (size 2.5 2.5) (drill 1.3) (layers *.Cu *.Mask) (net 9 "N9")))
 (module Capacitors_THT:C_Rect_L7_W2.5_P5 (layer F.Cu) (at 199.39 78.74)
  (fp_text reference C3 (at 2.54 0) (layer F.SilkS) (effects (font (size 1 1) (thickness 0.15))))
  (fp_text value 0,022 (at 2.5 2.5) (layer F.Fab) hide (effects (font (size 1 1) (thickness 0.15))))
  (fp_line (start -1 -1.25) (end 6 -1.25) (layer F.SilkS) (width 0.15))
  (fp_line (start 6 -1.25) (end 6 1.25) (layer F.SilkS) (width 0.15))
  (fp_line (start 6 1.25) (end -1 1.25) (layer F.SilkS) (width 0.15))
  (fp_line (start -1 1.25) (end -1 -1.25) (layer F.SilkS) (width 0.15))
  (pad 1 thru_hole rect (at 0 0) (size 1.3 1.3) (drill 0.8) (layers *.Cu *.Mask) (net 9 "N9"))
  (pad 2 thru_hole circle (at 5 0) (size 1.3 1.3) (drill 0.8) (layers *.Cu *.Mask) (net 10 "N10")))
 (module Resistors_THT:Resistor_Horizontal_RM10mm (layer F.Cu) (at 208.28 78.74)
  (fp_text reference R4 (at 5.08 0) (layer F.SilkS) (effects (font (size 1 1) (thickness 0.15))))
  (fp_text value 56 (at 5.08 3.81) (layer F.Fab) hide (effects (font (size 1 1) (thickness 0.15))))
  (fp_line (start 2.54 -1.27) (end 7.62 -1.27) (layer F.SilkS) (width 0.15))
  (fp_line (start 7.62 -1.27) (end 7.62 1.27) (layer F.SilkS) (width 0.15))
  (fp_line (start 7.62 1.27) (end 2.54 1.27) (layer F.SilkS) (width 0.15))
  (fp_line (start 2.54 1.27) (end 2.54 -1.27) (layer F.SilkS) (width 0.15))
  (fp_line (start 2.54 0) (end 1.27 0) (layer F.SilkS) (width 0.15))
  (fp_line (start 7.62 0) (end 8.89 0) (layer F.SilkS) (width 0.15))
  (pad 1 thru_hole circle (at 0 0) (size 1.99898 1.99898) (drill 1.00076) (layers *.Cu *.SilkS *.Mask) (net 10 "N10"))
  (pad 2 thru_hole circle (at 10.16 0) (size 1.99898 1.99898) (drill 1.00076) (layers *.Cu *.SilkS *.Mask) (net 8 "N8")))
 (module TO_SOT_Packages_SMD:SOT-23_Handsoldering (layer B.Cu) (at 189.23 81.28)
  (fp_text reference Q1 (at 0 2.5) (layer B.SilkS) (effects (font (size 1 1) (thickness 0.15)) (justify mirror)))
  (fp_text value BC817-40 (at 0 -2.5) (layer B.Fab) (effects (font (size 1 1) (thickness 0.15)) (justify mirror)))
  (pad 1 smd rect (at -1.5 0.95) (size 1.9 0.8) (layers B.Cu B.Paste B.Mask) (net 6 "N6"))
  (pad 2 smd rect (at -1.5 -0.95) (size 1.9 0.8) (layers B.Cu B.Paste B.Mask) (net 3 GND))
  (pad 3 smd rect (at 1.5 0) (size 1.9 0.8) (layers B.Cu B.Paste B.Mask) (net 2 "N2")))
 (gr_circle (center 226.06 78.74) (end 227.33 78.74) (layer Edge.Cuts) (width 0.15))
 (gr_circle (center 226.06 95.25) (end 227.33 95.25) (layer Edge.Cuts) (width 0.15))
 (gr_circle (center 176.53 95.25) (end 177.8 95.25) (layer Edge.Cuts) (width 0.15))
 (gr_circle (center 176.53 78.74) (end 177.8 78.74) (layer Edge.Cuts) (width 0.15))
 (gr_circle (center 176.53 78.74) (end 175.26 78.74) (layer F.SilkS) (width 0.2))
 (gr_circle (center 176.53 95.25) (end 175.26 95.25) (layer F.SilkS) (width 0.2))
 (gr_circle (center 226.06 78.74) (end 227.33 78.74) (layer F.SilkS) (width 0.2))
 (gr_circle (center 226.06 95.25) (end 226.06 96.52) (layer F.SilkS) (width 0.2))
 (gr_line (start 173.99 76.2) (end 173.99 97.79) (angle 90) (layer Edge.Cuts) (width 0.15))
 (gr_line (start 229.87 76.2) (end 173.99 76.2) (angle 90) (layer Edge.Cuts) (width 0.15))
 (gr_line (start 229.87 97.79) (end 229.87 76.2) (angle 90) (layer Edge.Cuts) (width 0.15))
 (gr_line (start 173.99 97.79) (end 229.87 97.79) (angle 90) (layer Edge.Cuts) (width 0.15))
 (segment (start 194.99 94.95) (end 194.61 94.95) (width 0.25) (layer B.Cu) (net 1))
 (segment (start 194.61 94.95) (end 194.31 95.25) (width 0.25) (layer B.Cu) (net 1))
 (segment (start 194.31 95.25) (end 189.23 95.25) (width 0.4) (layer B.Cu) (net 1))
 (segment (start 189.23 95.25) (end 187.96 93.98) (width 0.4) (layer B.Cu) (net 1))
 (segment (start 187.96 93.98) (end 187.96 92.71) (width 0.25) (layer B.Cu) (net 1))
 (segment (start 186.69 95.25) (end 187.96 93.98) (width 0.25) (layer B.Cu) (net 1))
 (segment (start 181.61 95.25) (end 186.69 95.25) (width 0.25) (layer B.Cu) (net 1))
 (segment (start 181.61 87.63) (end 181.61 95.25) (width 0.25) (layer B.Cu) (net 1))
 (segment (start 179.07 87.63) (end 181.61 87.63) (width 0.25) (layer B.Cu) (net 1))
 (segment (start 179.023199 87.583199) (end 179.07 87.63) (width 0.25) (layer B.Cu) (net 1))
 (segment (start 179.023199 83.866801) (end 179.023199 87.583199) (width 0.25) (layer B.Cu) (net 1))
 (segment (start 179.07 83.82) (end 179.023199 83.866801) (width 0.25) (layer B.Cu) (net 1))
 (segment (start 181.61 83.82) (end 179.07 83.82) (width 0.25) (layer B.Cu) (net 1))
 (segment (start 182.88 82.55) (end 181.61 83.82) (width 0.25) (layer B.Cu) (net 1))
 (segment (start 183.61 82.55) (end 182.88 82.55) (width 0.25) (layer B.Cu) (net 1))
 (segment (start 183.61 82.55) (end 184.15 82.55) (width 0.25) (layer B.Cu) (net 1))
 (segment (start 187.96 88.9) (end 187.96 89.265) (width 0.25) (layer B.Cu) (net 1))
 (segment (start 183.261 80.01) (end 183.261 82.201) (width 0.4) (layer B.Cu) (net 1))
 (segment (start 183.261 82.201) (end 183.61 82.55) (width 0.25) (layer B.Cu) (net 1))
 (segment (start 187.96 89.265) (end 187.96 92.71) (width 0.4) (layer B.Cu) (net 1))
 (segment (start 179.61 82.55) (end 179.07 82.55) (width 0.25) (layer B.Cu) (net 3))
 (segment (start 179.07 82.55) (end 177.8 83.82) (width 0.4) (layer B.Cu) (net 3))
 (segment (start 177.8 87.09) (end 180.34 89.63) (width 0.25) (layer B.Cu) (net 3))
 (segment (start 177.8 83.82) (end 177.8 87.09) (width 0.4) (layer B.Cu) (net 3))
 (segment (start 179.959 80.01) (end 179.959 79.121) (width 0.25) (layer B.Cu) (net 3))
 (segment (start 179.959 79.121) (end 181.61 77.47) (width 0.25) (layer B.Cu) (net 3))
 (segment (start 188.23 79.01) (end 188.23 80.33) (width 0.4) (layer B.Cu) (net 3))
 (segment (start 186.69 77.47) (end 188.23 79.01) (width 0.4) (layer B.Cu) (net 3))
 (segment (start 181.61 77.47) (end 186.69 77.47) (width 0.4) (layer B.Cu) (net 3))
 (segment (start 179.959 80.01) (end 179.959 82.201) (width 0.4) (layer B.Cu) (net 3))
 (segment (start 179.959 82.201) (end 179.61 82.55) (width 0.25) (layer B.Cu) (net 3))
 (segment (start 180.34 89.63) (end 180.34 92.71) (width 0.4) (layer B.Cu) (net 3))
 (segment (start 190.23 81.28) (end 193.32 81.28) (width 0.4) (layer B.Cu) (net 2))
 (segment (start 193.32 81.28) (end 194.99 82.95) (width 0.4) (layer B.Cu) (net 2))
 (segment (start 190.23 81.28) (end 190.23 83.725) (width 0.4) (layer B.Cu) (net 2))
 (segment (start 190.23 83.725) (end 187.96 85.995) (width 0.4) (layer B.Cu) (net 2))
 (segment (start 185.42 85.63) (end 187.595 85.63) (width 0.4) (layer B.Cu) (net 2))
 (segment (start 187.595 85.63) (end 187.96 85.995) (width 0.25) (layer B.Cu) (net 2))
 (segment (start 182.88 89.63) (end 182.88 92.71) (width 0.4) (layer B.Cu) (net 5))
 (segment (start 184.15 83.82) (end 186.64 83.82) (width 0.25) (layer B.Cu) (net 6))
 (segment (start 182.88 85.63) (end 182.88 85.09) (width 0.25) (layer B.Cu) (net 6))
 (segment (start 182.88 85.09) (end 184.15 83.82) (width 0.25) (layer B.Cu) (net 6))
 (segment (start 186.64 83.82) (end 188.23 82.23) (width 0.25) (layer B.Cu) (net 6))
 (segment (start 180.34 85.63) (end 182.88 85.63) (width 0.25) (layer B.Cu) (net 6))
 (segment (start 185.42 89.63) (end 185.42 92.71) (width 0.4) (layer B.Cu) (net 4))
 (segment (start 218.44 83.98) (end 218.44 78.74) (width 2) (layer B.Cu) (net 8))
 (segment (start 207.24 82.9) (end 217.36 82.9) (width 2) (layer B.Cu) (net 8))
 (segment (start 217.36 82.9) (end 218.44 83.98) (width 2) (layer B.Cu) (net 8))
 (segment (start 207.19 94.95) (end 217.47 94.95) (width 2) (layer B.Cu) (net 7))
 (segment (start 217.47 94.95) (end 218.44 93.98) (width 2) (layer B.Cu) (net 7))
 (segment (start 199.39 78.74) (end 199.39 86.36) (width 2) (layer B.Cu) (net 9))
 (segment (start 199.39 86.36) (end 201.93 88.9) (width 2) (layer B.Cu) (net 9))
 (segment (start 193.04 88.9) (end 201.93 88.9) (width 2) (layer B.Cu) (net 9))
 (segment (start 201.93 88.9) (end 218.36 88.9) (width 2) (layer B.Cu) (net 9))
 (segment (start 218.36 88.9) (end 218.44 88.98) (width 0.25) (layer B.Cu) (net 9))
 (segment (start 204.39 78.74) (end 208.28 78.74) (width 2) (layer B.Cu) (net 10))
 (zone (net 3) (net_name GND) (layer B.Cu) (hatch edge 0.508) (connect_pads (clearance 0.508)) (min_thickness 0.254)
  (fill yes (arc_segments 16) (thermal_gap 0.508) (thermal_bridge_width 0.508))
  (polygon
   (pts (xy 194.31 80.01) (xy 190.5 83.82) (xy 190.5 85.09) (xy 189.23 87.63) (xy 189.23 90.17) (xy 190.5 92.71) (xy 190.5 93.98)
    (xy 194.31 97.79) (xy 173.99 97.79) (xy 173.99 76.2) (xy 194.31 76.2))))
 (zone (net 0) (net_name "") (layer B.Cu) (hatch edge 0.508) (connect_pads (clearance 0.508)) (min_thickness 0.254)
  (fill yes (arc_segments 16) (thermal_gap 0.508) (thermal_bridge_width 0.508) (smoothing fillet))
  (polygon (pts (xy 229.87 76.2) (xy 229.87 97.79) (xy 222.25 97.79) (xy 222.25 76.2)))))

